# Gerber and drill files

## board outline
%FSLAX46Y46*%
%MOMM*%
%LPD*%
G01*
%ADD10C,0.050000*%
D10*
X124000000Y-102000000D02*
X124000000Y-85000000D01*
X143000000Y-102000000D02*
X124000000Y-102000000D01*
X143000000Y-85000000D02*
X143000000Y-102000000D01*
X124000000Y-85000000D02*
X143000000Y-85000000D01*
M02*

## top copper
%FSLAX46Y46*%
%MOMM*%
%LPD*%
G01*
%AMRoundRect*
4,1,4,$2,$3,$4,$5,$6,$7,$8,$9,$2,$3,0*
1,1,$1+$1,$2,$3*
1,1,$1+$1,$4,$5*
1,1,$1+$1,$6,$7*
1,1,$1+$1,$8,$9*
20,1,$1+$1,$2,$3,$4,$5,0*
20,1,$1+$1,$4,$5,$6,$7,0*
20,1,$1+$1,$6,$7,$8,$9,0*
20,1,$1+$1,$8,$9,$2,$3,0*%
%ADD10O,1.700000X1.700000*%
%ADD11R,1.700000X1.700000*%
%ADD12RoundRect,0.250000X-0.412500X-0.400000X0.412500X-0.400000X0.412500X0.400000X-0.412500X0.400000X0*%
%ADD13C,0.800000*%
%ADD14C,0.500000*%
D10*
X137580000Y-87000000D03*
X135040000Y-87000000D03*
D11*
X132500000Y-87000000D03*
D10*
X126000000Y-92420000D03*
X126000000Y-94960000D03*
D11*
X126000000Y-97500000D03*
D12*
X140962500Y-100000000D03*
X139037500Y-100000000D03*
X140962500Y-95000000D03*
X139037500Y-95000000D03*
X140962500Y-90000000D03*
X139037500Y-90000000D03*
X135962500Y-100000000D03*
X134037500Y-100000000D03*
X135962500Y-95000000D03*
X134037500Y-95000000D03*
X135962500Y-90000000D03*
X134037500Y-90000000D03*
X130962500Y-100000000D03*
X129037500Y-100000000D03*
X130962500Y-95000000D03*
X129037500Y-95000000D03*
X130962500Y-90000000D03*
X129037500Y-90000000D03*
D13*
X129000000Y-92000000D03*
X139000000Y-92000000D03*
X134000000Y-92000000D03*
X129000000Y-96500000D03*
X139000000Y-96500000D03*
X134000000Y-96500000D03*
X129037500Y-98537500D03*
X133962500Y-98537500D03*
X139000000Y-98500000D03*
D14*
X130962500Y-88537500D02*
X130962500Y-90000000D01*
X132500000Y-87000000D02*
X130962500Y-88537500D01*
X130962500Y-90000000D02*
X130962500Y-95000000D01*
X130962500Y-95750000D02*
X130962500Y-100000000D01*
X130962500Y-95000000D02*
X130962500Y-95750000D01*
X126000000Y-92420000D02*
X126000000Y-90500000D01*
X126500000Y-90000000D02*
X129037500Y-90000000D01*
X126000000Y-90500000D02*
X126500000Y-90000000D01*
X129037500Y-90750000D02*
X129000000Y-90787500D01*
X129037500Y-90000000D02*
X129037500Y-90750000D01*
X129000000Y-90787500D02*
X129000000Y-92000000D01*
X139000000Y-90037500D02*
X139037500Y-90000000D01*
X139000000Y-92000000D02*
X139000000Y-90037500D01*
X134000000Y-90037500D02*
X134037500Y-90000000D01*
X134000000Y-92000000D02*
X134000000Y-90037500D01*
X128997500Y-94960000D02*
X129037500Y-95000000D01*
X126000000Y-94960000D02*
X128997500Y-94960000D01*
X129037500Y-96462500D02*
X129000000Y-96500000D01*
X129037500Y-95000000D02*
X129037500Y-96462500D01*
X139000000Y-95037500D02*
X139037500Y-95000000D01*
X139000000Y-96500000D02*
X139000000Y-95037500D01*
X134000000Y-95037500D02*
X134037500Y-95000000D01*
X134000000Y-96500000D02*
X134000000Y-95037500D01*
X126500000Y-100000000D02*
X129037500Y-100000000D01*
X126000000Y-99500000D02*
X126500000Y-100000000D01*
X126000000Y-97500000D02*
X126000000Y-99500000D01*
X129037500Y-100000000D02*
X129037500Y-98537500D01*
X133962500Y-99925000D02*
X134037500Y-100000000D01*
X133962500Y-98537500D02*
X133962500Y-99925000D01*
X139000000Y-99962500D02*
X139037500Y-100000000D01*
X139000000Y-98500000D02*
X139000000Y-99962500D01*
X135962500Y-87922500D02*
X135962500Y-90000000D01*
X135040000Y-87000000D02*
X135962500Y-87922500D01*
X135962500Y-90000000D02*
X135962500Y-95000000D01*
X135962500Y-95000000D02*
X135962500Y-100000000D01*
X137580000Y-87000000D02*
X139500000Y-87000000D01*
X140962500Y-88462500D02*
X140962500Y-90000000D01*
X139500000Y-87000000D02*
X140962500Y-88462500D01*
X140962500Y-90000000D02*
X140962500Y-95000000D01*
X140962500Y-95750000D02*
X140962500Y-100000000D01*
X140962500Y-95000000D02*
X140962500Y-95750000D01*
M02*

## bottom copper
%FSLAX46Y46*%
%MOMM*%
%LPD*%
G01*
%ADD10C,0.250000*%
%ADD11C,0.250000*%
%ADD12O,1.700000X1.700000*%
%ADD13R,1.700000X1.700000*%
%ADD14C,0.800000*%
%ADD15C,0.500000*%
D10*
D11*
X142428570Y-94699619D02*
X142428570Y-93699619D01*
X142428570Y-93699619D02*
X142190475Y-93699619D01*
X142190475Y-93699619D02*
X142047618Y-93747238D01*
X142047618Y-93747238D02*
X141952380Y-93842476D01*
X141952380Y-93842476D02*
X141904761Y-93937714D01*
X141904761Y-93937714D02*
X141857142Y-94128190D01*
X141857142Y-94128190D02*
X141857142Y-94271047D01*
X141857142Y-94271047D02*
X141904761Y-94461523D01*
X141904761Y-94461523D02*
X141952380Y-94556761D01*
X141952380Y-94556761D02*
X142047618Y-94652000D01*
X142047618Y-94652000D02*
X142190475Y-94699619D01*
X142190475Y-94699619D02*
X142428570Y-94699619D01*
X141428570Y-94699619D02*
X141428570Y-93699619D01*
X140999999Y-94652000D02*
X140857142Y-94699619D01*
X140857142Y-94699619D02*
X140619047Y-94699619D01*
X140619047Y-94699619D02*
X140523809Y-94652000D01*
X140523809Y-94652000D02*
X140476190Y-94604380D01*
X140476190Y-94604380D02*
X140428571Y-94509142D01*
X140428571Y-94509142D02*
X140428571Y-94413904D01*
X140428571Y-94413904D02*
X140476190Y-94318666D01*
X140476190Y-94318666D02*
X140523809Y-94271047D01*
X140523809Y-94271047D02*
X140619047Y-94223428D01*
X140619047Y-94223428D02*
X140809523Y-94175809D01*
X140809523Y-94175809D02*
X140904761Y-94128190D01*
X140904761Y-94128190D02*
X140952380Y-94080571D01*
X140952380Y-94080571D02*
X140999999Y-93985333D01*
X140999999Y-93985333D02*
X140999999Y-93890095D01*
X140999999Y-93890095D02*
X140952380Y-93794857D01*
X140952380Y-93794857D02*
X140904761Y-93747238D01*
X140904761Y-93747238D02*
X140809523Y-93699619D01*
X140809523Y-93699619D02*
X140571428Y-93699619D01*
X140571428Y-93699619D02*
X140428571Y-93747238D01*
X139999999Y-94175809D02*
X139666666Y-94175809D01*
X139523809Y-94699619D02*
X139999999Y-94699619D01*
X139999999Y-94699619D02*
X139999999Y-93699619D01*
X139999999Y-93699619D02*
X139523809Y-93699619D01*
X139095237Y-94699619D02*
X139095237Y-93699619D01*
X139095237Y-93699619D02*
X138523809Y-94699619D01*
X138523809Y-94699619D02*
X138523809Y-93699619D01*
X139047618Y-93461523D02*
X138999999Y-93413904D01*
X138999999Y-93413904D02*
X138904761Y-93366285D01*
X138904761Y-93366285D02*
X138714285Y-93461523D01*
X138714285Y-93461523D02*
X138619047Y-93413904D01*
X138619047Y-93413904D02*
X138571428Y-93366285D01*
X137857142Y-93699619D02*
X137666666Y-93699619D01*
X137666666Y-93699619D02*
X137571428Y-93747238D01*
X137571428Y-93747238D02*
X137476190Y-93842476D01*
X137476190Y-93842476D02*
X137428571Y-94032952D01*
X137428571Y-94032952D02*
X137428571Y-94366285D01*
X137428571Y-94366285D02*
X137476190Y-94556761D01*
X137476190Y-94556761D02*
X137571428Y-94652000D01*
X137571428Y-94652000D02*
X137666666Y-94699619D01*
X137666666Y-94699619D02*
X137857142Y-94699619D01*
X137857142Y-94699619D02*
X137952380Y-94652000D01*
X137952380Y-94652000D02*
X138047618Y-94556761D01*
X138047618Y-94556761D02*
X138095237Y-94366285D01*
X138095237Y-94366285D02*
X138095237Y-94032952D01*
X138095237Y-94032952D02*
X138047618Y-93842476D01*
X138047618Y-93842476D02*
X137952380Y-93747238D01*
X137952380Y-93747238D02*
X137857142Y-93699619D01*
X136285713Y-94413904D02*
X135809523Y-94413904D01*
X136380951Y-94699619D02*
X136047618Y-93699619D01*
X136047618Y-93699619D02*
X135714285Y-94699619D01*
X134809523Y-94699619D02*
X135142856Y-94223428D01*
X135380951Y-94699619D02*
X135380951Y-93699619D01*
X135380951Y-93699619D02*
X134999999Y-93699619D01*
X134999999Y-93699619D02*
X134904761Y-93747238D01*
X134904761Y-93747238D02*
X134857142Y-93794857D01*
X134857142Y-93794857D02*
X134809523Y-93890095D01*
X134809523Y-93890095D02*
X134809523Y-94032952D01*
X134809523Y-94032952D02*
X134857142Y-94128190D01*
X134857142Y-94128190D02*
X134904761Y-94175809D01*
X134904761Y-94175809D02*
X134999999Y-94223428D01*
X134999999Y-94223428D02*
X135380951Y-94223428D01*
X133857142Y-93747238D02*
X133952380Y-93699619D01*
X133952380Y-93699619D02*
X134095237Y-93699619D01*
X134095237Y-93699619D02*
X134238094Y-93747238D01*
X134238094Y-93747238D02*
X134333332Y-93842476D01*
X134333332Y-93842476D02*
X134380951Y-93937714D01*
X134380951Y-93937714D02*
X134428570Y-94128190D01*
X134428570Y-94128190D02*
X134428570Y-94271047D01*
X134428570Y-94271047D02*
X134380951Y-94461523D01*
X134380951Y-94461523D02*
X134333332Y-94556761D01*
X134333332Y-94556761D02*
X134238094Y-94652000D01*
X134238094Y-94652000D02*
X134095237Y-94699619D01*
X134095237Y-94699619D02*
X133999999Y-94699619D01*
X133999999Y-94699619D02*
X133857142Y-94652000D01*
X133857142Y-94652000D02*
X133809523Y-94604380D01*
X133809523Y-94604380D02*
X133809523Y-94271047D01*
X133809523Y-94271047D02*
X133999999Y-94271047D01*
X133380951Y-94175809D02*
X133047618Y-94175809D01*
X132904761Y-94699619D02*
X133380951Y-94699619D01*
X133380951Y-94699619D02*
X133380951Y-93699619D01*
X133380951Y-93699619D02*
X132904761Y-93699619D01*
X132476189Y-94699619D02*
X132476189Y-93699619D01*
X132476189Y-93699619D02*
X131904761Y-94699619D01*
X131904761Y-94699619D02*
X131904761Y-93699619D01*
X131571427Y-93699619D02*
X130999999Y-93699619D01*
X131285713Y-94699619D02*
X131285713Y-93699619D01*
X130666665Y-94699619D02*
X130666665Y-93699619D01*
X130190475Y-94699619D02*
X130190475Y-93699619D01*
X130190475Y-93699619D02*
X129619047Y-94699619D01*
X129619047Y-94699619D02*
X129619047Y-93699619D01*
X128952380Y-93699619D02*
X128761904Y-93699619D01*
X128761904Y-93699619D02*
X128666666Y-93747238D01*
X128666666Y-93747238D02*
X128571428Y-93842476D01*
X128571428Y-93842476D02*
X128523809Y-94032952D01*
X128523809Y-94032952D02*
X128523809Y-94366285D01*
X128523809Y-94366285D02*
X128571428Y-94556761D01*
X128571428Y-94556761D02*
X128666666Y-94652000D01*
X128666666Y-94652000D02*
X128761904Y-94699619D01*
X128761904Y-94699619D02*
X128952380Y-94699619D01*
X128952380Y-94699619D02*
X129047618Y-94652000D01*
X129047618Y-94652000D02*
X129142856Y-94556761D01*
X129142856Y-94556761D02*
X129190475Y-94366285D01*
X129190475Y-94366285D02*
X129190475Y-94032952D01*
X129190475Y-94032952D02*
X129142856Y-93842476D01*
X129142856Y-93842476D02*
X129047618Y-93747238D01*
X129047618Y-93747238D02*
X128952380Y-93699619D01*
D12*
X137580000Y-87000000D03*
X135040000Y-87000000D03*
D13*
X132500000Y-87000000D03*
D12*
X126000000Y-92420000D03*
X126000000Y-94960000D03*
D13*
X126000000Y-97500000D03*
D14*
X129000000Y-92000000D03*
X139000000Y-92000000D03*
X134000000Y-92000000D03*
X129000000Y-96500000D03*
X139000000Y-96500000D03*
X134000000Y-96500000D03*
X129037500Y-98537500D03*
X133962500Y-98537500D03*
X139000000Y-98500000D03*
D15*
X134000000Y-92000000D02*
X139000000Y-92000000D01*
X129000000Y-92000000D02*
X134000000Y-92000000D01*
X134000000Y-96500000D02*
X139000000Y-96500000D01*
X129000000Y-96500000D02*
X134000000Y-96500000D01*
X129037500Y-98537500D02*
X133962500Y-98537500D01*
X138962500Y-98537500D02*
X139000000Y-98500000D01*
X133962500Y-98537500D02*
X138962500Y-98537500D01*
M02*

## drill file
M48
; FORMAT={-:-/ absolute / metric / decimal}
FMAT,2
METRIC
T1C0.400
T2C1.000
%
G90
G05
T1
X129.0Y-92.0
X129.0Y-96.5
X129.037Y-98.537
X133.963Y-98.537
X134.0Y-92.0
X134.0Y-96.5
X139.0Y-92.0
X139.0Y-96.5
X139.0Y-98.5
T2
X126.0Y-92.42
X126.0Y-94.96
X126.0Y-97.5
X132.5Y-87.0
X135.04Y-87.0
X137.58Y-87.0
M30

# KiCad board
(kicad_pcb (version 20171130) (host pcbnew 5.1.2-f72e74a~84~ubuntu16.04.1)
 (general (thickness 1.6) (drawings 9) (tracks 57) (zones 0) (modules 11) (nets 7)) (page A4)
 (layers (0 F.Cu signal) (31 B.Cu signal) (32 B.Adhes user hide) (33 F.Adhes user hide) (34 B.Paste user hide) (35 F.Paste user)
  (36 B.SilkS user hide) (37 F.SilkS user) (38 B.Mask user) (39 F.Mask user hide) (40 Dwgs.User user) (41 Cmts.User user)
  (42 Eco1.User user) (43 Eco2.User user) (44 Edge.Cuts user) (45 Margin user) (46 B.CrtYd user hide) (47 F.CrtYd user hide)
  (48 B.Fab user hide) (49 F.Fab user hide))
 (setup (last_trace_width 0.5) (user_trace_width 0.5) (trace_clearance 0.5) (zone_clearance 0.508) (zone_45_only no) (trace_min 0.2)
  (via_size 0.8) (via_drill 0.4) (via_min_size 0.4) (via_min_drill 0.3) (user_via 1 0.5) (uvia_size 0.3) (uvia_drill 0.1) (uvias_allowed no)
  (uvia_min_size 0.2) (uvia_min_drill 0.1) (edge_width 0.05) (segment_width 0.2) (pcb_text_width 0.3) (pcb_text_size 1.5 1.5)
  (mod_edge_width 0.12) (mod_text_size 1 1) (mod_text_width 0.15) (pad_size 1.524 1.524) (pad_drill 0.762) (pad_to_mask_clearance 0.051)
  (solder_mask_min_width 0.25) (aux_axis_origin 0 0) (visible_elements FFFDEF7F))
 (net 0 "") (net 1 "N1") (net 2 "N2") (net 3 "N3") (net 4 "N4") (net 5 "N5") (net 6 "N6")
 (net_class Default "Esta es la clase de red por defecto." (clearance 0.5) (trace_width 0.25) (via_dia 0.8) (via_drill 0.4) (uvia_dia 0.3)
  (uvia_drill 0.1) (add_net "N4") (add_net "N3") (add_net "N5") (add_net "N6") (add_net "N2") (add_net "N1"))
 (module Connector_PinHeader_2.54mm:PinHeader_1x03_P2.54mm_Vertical (layer B.Cu) (at 132.5 87 270)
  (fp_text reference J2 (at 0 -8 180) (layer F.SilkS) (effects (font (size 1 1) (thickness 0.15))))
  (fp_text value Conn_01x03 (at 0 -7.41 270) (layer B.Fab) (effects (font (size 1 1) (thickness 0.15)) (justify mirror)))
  (pad 3 thru_hole oval (at 0 -5.08 270) (size 1.7 1.7) (drill 1) (layers *.Cu *.Mask) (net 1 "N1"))
  (pad 2 thru_hole oval (at 0 -2.54 270) (size 1.7 1.7) (drill 1) (layers *.Cu *.Mask) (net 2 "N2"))
  (pad 1 thru_hole rect (at 0 0 270) (size 1.7 1.7) (drill 1) (layers *.Cu *.Mask) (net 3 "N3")))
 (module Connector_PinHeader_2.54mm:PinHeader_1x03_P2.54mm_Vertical (layer B.Cu) (at 126 97.5)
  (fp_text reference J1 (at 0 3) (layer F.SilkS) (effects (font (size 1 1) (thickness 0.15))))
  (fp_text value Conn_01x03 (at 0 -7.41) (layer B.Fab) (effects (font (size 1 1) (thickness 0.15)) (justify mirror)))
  (pad 3 thru_hole oval (at 0 -5.08) (size 1.7 1.7) (drill 1) (layers *.Cu *.Mask) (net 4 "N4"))
  (pad 2 thru_hole oval (at 0 -2.54) (size 1.7 1.7) (drill 1) (layers *.Cu *.Mask) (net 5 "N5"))
  (pad 1 thru_hole rect (at 0 0) (size 1.7 1.7) (drill 1) (layers *.Cu *.Mask) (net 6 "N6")))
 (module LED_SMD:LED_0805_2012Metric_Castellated (layer F.Cu) (at 140 100)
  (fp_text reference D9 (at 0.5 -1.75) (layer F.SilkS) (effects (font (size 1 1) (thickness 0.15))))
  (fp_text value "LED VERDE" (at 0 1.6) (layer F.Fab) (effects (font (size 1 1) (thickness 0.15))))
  (pad 2 smd roundrect (at 0.9625 0) (size 1.325 1.3) (layers F.Cu F.Paste F.Mask) (roundrect_rratio 0.192308) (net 1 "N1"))
  (pad 1 smd roundrect (at -0.9625 0) (size 1.325 1.3) (layers F.Cu F.Paste F.Mask) (roundrect_rratio 0.192308) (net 6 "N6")))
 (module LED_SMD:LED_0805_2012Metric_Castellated (layer F.Cu) (at 140 95)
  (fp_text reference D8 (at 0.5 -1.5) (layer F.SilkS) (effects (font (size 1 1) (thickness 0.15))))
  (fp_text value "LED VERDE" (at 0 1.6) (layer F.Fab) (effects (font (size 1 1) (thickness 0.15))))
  (pad 2 smd roundrect (at 0.9625 0) (size 1.325 1.3) (layers F.Cu F.Paste F.Mask) (roundrect_rratio 0.192308) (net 1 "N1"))
  (pad 1 smd roundrect (at -0.9625 0) (size 1.325 1.3) (layers F.Cu F.Paste F.Mask) (roundrect_rratio 0.192308) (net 5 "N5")))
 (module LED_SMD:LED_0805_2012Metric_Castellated (layer F.Cu) (at 140 90)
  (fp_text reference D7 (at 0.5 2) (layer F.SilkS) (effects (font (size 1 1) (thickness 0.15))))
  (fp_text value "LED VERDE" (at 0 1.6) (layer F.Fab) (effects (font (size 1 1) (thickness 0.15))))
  (pad 2 smd roundrect (at 0.9625 0) (size 1.325 1.3) (layers F.Cu F.Paste F.Mask) (roundrect_rratio 0.192308) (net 1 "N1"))
  (pad 1 smd roundrect (at -0.9625 0) (size 1.325 1.3) (layers F.Cu F.Paste F.Mask) (roundrect_rratio 0.192308) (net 4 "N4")))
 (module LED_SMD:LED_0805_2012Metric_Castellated (layer F.Cu) (at 135 100)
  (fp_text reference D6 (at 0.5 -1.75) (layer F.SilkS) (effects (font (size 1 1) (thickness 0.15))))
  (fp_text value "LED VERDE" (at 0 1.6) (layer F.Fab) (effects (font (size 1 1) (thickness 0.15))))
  (pad 2 smd roundrect (at 0.9625 0) (size 1.325 1.3) (layers F.Cu F.Paste F.Mask) (roundrect_rratio 0.192308) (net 2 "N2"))
  (pad 1 smd roundrect (at -0.9625 0) (size 1.325 1.3) (layers F.Cu F.Paste F.Mask) (roundrect_rratio 0.192308) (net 6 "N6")))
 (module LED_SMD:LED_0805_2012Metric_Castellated (layer F.Cu) (at 135 95)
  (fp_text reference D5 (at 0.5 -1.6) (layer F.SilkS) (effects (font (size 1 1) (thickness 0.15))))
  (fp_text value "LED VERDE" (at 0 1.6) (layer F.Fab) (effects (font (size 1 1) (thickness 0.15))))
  (pad 2 smd roundrect (at 0.9625 0) (size 1.325 1.3) (layers F.Cu F.Paste F.Mask) (roundrect_rratio 0.192308) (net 2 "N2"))
  (pad 1 smd roundrect (at -0.9625 0) (size 1.325 1.3) (layers F.Cu F.Paste F.Mask) (roundrect_rratio 0.192308) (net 5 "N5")))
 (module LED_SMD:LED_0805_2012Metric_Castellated (layer F.Cu) (at 135 90)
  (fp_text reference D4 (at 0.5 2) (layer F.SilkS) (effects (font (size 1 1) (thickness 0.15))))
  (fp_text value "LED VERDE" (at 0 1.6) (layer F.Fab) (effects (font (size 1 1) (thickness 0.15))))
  (pad 2 smd roundrect (at 0.9625 0) (size 1.325 1.3) (layers F.Cu F.Paste F.Mask) (roundrect_rratio 0.192308) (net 2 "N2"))
  (pad 1 smd roundrect (at -0.9625 0) (size 1.325 1.3) (layers F.Cu F.Paste F.Mask) (roundrect_rratio 0.192308) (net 4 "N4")))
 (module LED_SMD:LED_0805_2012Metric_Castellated (layer F.Cu) (at 130 100)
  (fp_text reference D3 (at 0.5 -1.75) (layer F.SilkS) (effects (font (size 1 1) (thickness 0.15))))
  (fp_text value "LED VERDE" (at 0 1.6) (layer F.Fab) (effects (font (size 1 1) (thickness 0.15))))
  (pad 2 smd roundrect (at 0.9625 0) (size 1.325 1.3) (layers F.Cu F.Paste F.Mask) (roundrect_rratio 0.192308) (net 3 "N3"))
  (pad 1 smd roundrect (at -0.9625 0) (size 1.325 1.3) (layers F.Cu F.Paste F.Mask) (roundrect_rratio 0.192308) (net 6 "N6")))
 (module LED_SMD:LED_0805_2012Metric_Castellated (layer F.Cu) (at 130 95)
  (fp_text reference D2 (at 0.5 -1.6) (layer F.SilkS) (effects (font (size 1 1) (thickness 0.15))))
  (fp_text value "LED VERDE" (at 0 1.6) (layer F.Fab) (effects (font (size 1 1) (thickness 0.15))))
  (pad 2 smd roundrect (at 0.9625 0) (size 1.325 1.3) (layers F.Cu F.Paste F.Mask) (roundrect_rratio 0.192308) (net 3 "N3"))
  (pad 1 smd roundrect (at -0.9625 0) (size 1.325 1.3) (layers F.Cu F.Paste F.Mask) (roundrect_rratio 0.192308) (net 5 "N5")))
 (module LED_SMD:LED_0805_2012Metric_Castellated (layer F.Cu) (at 130 90)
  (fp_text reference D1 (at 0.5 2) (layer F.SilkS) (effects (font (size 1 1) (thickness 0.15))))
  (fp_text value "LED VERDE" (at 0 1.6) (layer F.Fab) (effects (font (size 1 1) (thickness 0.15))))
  (pad 2 smd roundrect (at 0.9625 0) (size 1.325 1.3) (layers F.Cu F.Paste F.Mask) (roundrect_rratio 0.192308) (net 3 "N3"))
  (pad 1 smd roundrect (at -0.9625 0) (size 1.325 1.3) (layers F.Cu F.Paste F.Mask) (roundrect_rratio 0.192308) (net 4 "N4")))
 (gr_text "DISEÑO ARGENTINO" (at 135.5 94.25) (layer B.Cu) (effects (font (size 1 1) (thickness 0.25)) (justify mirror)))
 (gr_line (start 124 102) (end 124 85) (layer Edge.Cuts) (width 0.05))
 (gr_line (start 143 102) (end 124 102) (layer Edge.Cuts) (width 0.05))
 (gr_line (start 143 85) (end 143 102) (layer Edge.Cuts) (width 0.05))
 (gr_line (start 124 85) (end 143 85) (layer Edge.Cuts) (width 0.05))
 (segment (start 130.9625 88.5375) (end 130.9625 90) (width 0.5) (layer F.Cu) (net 3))
 (segment (start 132.5 87) (end 130.9625 88.5375) (width 0.5) (layer F.Cu) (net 3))
 (segment (start 130.9625 90) (end 130.9625 95) (width 0.5) (layer F.Cu) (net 3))
 (segment (start 130.9625 95.75) (end 130.9625 100) (width 0.5) (layer F.Cu) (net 3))
 (segment (start 130.9625 95) (end 130.9625 95.75) (width 0.5) (layer F.Cu) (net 3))
 (segment (start 126 92.42) (end 126 90.5) (width 0.5) (layer F.Cu) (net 4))
 (segment (start 126.5 90) (end 129.0375 90) (width 0.5) (layer F.Cu) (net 4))
 (segment (start 126 90.5) (end 126.5 90) (width 0.5) (layer F.Cu) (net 4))
 (segment (start 129.0375 90.75) (end 129 90.7875) (width 0.5) (layer F.Cu) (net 4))
 (segment (start 129.0375 90) (end 129.0375 90.75) (width 0.5) (layer F.Cu) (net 4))
 (via (at 129 92) (size 0.8) (drill 0.4) (layers F.Cu B.Cu) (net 4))
 (segment (start 129 90.7875) (end 129 92) (width 0.5) (layer F.Cu) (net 4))
 (via (at 139 92) (size 0.8) (drill 0.4) (layers F.Cu B.Cu) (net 4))
 (segment (start 139 90.0375) (end 139.0375 90) (width 0.5) (layer F.Cu) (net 4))
 (segment (start 139 92) (end 139 90.0375) (width 0.5) (layer F.Cu) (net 4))
 (segment (start 134 92) (end 139 92) (width 0.5) (layer B.Cu) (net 4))
 (segment (start 129 92) (end 134 92) (width 0.5) (layer B.Cu) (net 4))
 (via (at 134 92) (size 0.8) (drill 0.4) (layers F.Cu B.Cu) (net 4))
 (segment (start 134 90.0375) (end 134.0375 90) (width 0.5) (layer F.Cu) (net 4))
 (segment (start 134 92) (end 134 90.0375) (width 0.5) (layer F.Cu) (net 4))
 (segment (start 128.9975 94.96) (end 129.0375 95) (width 0.5) (layer F.Cu) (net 5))
 (segment (start 126 94.96) (end 128.9975 94.96) (width 0.5) (layer F.Cu) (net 5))
 (via (at 129 96.5) (size 0.8) (drill 0.4) (layers F.Cu B.Cu) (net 5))
 (segment (start 129.0375 96.4625) (end 129 96.5) (width 0.5) (layer F.Cu) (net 5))
 (segment (start 129.0375 95) (end 129.0375 96.4625) (width 0.5) (layer F.Cu) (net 5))
 (via (at 139 96.5) (size 0.8) (drill 0.4) (layers F.Cu B.Cu) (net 5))
 (segment (start 139 95.0375) (end 139.0375 95) (width 0.5) (layer F.Cu) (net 5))
 (segment (start 139 96.5) (end 139 95.0375) (width 0.5) (layer F.Cu) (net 5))
 (segment (start 134 96.5) (end 139 96.5) (width 0.5) (layer B.Cu) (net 5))
 (segment (start 129 96.5) (end 134 96.5) (width 0.5) (layer B.Cu) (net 5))
 (via (at 134 96.5) (size 0.8) (drill 0.4) (layers F.Cu B.Cu) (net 5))
 (segment (start 134 95.0375) (end 134.0375 95) (width 0.5) (layer F.Cu) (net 5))
 (segment (start 134 96.5) (end 134 95.0375) (width 0.5) (layer F.Cu) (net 5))
 (segment (start 126.5 100) (end 129.0375 100) (width 0.5) (layer F.Cu) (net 6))
 (segment (start 126 99.5) (end 126.5 100) (width 0.5) (layer F.Cu) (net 6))
 (segment (start 126 97.5) (end 126 99.5) (width 0.5) (layer F.Cu) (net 6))
 (segment (start 129.0375 100) (end 129.0375 98.5375) (width 0.5) (layer F.Cu) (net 6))
 (via (at 129.0375 98.5375) (size 0.8) (drill 0.4) (layers F.Cu B.Cu) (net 6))
 (segment (start 129.0375 98.5375) (end 133.9625 98.5375) (width 0.5) (layer B.Cu) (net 6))
 (via (at 133.9625 98.5375) (size 0.8) (drill 0.4) (layers F.Cu B.Cu) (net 6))
 (segment (start 133.9625 99.925) (end 134.0375 100) (width 0.5) (layer F.Cu) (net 6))
 (segment (start 133.9625 98.5375) (end 133.9625 99.925) (width 0.5) (layer F.Cu) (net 6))
 (segment (start 138.9625 98.5375) (end 139 98.5) (width 0.5) (layer B.Cu) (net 6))
 (via (at 139 98.5) (size 0.8) (drill 0.4) (layers F.Cu B.Cu) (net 6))
 (segment (start 133.9625 98.5375) (end 138.9625 98.5375) (width 0.5) (layer B.Cu) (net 6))
 (segment (start 139 99.9625) (end 139.0375 100) (width 0.5) (layer F.Cu) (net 6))
 (segment (start 139 98.5) (end 139 99.9625) (width 0.5) (layer F.Cu) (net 6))
 (segment (start 135.9625 87.9225) (end 135.9625 90) (width 0.5) (layer F.Cu) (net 2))
 (segment (start 135.04 87) (end 135.9625 87.9225) (width 0.5) (layer F.Cu) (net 2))
 (segment (start 135.9625 90) (end 135.9625 95) (width 0.5) (layer F.Cu) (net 2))
 (segment (start 135.9625 95) (end 135.9625 100) (width 0.5) (layer F.Cu) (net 2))
 (segment (start 137.58 87) (end 139.5 87) (width 0.5) (layer F.Cu) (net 1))
 (segment (start 140.9625 88.4625) (end 140.9625 90) (width 0.5) (layer F.Cu) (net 1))
 (segment (start 139.5 87) (end 140.9625 88.4625) (width 0.5) (layer F.Cu) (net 1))
 (segment (start 140.9625 90) (end 140.9625 95) (width 0.5) (layer F.Cu) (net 1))
 (segment (start 140.9625 95.75) (end 140.9625 100) (width 0.5) (layer F.Cu) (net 1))
 (segment (start 140.9625 95) (end 140.9625 95.75) (width 0.5) (layer F.Cu) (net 1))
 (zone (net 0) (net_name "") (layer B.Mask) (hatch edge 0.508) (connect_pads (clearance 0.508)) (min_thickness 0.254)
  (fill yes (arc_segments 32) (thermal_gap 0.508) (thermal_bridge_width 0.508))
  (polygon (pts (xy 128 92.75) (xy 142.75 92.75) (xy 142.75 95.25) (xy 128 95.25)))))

